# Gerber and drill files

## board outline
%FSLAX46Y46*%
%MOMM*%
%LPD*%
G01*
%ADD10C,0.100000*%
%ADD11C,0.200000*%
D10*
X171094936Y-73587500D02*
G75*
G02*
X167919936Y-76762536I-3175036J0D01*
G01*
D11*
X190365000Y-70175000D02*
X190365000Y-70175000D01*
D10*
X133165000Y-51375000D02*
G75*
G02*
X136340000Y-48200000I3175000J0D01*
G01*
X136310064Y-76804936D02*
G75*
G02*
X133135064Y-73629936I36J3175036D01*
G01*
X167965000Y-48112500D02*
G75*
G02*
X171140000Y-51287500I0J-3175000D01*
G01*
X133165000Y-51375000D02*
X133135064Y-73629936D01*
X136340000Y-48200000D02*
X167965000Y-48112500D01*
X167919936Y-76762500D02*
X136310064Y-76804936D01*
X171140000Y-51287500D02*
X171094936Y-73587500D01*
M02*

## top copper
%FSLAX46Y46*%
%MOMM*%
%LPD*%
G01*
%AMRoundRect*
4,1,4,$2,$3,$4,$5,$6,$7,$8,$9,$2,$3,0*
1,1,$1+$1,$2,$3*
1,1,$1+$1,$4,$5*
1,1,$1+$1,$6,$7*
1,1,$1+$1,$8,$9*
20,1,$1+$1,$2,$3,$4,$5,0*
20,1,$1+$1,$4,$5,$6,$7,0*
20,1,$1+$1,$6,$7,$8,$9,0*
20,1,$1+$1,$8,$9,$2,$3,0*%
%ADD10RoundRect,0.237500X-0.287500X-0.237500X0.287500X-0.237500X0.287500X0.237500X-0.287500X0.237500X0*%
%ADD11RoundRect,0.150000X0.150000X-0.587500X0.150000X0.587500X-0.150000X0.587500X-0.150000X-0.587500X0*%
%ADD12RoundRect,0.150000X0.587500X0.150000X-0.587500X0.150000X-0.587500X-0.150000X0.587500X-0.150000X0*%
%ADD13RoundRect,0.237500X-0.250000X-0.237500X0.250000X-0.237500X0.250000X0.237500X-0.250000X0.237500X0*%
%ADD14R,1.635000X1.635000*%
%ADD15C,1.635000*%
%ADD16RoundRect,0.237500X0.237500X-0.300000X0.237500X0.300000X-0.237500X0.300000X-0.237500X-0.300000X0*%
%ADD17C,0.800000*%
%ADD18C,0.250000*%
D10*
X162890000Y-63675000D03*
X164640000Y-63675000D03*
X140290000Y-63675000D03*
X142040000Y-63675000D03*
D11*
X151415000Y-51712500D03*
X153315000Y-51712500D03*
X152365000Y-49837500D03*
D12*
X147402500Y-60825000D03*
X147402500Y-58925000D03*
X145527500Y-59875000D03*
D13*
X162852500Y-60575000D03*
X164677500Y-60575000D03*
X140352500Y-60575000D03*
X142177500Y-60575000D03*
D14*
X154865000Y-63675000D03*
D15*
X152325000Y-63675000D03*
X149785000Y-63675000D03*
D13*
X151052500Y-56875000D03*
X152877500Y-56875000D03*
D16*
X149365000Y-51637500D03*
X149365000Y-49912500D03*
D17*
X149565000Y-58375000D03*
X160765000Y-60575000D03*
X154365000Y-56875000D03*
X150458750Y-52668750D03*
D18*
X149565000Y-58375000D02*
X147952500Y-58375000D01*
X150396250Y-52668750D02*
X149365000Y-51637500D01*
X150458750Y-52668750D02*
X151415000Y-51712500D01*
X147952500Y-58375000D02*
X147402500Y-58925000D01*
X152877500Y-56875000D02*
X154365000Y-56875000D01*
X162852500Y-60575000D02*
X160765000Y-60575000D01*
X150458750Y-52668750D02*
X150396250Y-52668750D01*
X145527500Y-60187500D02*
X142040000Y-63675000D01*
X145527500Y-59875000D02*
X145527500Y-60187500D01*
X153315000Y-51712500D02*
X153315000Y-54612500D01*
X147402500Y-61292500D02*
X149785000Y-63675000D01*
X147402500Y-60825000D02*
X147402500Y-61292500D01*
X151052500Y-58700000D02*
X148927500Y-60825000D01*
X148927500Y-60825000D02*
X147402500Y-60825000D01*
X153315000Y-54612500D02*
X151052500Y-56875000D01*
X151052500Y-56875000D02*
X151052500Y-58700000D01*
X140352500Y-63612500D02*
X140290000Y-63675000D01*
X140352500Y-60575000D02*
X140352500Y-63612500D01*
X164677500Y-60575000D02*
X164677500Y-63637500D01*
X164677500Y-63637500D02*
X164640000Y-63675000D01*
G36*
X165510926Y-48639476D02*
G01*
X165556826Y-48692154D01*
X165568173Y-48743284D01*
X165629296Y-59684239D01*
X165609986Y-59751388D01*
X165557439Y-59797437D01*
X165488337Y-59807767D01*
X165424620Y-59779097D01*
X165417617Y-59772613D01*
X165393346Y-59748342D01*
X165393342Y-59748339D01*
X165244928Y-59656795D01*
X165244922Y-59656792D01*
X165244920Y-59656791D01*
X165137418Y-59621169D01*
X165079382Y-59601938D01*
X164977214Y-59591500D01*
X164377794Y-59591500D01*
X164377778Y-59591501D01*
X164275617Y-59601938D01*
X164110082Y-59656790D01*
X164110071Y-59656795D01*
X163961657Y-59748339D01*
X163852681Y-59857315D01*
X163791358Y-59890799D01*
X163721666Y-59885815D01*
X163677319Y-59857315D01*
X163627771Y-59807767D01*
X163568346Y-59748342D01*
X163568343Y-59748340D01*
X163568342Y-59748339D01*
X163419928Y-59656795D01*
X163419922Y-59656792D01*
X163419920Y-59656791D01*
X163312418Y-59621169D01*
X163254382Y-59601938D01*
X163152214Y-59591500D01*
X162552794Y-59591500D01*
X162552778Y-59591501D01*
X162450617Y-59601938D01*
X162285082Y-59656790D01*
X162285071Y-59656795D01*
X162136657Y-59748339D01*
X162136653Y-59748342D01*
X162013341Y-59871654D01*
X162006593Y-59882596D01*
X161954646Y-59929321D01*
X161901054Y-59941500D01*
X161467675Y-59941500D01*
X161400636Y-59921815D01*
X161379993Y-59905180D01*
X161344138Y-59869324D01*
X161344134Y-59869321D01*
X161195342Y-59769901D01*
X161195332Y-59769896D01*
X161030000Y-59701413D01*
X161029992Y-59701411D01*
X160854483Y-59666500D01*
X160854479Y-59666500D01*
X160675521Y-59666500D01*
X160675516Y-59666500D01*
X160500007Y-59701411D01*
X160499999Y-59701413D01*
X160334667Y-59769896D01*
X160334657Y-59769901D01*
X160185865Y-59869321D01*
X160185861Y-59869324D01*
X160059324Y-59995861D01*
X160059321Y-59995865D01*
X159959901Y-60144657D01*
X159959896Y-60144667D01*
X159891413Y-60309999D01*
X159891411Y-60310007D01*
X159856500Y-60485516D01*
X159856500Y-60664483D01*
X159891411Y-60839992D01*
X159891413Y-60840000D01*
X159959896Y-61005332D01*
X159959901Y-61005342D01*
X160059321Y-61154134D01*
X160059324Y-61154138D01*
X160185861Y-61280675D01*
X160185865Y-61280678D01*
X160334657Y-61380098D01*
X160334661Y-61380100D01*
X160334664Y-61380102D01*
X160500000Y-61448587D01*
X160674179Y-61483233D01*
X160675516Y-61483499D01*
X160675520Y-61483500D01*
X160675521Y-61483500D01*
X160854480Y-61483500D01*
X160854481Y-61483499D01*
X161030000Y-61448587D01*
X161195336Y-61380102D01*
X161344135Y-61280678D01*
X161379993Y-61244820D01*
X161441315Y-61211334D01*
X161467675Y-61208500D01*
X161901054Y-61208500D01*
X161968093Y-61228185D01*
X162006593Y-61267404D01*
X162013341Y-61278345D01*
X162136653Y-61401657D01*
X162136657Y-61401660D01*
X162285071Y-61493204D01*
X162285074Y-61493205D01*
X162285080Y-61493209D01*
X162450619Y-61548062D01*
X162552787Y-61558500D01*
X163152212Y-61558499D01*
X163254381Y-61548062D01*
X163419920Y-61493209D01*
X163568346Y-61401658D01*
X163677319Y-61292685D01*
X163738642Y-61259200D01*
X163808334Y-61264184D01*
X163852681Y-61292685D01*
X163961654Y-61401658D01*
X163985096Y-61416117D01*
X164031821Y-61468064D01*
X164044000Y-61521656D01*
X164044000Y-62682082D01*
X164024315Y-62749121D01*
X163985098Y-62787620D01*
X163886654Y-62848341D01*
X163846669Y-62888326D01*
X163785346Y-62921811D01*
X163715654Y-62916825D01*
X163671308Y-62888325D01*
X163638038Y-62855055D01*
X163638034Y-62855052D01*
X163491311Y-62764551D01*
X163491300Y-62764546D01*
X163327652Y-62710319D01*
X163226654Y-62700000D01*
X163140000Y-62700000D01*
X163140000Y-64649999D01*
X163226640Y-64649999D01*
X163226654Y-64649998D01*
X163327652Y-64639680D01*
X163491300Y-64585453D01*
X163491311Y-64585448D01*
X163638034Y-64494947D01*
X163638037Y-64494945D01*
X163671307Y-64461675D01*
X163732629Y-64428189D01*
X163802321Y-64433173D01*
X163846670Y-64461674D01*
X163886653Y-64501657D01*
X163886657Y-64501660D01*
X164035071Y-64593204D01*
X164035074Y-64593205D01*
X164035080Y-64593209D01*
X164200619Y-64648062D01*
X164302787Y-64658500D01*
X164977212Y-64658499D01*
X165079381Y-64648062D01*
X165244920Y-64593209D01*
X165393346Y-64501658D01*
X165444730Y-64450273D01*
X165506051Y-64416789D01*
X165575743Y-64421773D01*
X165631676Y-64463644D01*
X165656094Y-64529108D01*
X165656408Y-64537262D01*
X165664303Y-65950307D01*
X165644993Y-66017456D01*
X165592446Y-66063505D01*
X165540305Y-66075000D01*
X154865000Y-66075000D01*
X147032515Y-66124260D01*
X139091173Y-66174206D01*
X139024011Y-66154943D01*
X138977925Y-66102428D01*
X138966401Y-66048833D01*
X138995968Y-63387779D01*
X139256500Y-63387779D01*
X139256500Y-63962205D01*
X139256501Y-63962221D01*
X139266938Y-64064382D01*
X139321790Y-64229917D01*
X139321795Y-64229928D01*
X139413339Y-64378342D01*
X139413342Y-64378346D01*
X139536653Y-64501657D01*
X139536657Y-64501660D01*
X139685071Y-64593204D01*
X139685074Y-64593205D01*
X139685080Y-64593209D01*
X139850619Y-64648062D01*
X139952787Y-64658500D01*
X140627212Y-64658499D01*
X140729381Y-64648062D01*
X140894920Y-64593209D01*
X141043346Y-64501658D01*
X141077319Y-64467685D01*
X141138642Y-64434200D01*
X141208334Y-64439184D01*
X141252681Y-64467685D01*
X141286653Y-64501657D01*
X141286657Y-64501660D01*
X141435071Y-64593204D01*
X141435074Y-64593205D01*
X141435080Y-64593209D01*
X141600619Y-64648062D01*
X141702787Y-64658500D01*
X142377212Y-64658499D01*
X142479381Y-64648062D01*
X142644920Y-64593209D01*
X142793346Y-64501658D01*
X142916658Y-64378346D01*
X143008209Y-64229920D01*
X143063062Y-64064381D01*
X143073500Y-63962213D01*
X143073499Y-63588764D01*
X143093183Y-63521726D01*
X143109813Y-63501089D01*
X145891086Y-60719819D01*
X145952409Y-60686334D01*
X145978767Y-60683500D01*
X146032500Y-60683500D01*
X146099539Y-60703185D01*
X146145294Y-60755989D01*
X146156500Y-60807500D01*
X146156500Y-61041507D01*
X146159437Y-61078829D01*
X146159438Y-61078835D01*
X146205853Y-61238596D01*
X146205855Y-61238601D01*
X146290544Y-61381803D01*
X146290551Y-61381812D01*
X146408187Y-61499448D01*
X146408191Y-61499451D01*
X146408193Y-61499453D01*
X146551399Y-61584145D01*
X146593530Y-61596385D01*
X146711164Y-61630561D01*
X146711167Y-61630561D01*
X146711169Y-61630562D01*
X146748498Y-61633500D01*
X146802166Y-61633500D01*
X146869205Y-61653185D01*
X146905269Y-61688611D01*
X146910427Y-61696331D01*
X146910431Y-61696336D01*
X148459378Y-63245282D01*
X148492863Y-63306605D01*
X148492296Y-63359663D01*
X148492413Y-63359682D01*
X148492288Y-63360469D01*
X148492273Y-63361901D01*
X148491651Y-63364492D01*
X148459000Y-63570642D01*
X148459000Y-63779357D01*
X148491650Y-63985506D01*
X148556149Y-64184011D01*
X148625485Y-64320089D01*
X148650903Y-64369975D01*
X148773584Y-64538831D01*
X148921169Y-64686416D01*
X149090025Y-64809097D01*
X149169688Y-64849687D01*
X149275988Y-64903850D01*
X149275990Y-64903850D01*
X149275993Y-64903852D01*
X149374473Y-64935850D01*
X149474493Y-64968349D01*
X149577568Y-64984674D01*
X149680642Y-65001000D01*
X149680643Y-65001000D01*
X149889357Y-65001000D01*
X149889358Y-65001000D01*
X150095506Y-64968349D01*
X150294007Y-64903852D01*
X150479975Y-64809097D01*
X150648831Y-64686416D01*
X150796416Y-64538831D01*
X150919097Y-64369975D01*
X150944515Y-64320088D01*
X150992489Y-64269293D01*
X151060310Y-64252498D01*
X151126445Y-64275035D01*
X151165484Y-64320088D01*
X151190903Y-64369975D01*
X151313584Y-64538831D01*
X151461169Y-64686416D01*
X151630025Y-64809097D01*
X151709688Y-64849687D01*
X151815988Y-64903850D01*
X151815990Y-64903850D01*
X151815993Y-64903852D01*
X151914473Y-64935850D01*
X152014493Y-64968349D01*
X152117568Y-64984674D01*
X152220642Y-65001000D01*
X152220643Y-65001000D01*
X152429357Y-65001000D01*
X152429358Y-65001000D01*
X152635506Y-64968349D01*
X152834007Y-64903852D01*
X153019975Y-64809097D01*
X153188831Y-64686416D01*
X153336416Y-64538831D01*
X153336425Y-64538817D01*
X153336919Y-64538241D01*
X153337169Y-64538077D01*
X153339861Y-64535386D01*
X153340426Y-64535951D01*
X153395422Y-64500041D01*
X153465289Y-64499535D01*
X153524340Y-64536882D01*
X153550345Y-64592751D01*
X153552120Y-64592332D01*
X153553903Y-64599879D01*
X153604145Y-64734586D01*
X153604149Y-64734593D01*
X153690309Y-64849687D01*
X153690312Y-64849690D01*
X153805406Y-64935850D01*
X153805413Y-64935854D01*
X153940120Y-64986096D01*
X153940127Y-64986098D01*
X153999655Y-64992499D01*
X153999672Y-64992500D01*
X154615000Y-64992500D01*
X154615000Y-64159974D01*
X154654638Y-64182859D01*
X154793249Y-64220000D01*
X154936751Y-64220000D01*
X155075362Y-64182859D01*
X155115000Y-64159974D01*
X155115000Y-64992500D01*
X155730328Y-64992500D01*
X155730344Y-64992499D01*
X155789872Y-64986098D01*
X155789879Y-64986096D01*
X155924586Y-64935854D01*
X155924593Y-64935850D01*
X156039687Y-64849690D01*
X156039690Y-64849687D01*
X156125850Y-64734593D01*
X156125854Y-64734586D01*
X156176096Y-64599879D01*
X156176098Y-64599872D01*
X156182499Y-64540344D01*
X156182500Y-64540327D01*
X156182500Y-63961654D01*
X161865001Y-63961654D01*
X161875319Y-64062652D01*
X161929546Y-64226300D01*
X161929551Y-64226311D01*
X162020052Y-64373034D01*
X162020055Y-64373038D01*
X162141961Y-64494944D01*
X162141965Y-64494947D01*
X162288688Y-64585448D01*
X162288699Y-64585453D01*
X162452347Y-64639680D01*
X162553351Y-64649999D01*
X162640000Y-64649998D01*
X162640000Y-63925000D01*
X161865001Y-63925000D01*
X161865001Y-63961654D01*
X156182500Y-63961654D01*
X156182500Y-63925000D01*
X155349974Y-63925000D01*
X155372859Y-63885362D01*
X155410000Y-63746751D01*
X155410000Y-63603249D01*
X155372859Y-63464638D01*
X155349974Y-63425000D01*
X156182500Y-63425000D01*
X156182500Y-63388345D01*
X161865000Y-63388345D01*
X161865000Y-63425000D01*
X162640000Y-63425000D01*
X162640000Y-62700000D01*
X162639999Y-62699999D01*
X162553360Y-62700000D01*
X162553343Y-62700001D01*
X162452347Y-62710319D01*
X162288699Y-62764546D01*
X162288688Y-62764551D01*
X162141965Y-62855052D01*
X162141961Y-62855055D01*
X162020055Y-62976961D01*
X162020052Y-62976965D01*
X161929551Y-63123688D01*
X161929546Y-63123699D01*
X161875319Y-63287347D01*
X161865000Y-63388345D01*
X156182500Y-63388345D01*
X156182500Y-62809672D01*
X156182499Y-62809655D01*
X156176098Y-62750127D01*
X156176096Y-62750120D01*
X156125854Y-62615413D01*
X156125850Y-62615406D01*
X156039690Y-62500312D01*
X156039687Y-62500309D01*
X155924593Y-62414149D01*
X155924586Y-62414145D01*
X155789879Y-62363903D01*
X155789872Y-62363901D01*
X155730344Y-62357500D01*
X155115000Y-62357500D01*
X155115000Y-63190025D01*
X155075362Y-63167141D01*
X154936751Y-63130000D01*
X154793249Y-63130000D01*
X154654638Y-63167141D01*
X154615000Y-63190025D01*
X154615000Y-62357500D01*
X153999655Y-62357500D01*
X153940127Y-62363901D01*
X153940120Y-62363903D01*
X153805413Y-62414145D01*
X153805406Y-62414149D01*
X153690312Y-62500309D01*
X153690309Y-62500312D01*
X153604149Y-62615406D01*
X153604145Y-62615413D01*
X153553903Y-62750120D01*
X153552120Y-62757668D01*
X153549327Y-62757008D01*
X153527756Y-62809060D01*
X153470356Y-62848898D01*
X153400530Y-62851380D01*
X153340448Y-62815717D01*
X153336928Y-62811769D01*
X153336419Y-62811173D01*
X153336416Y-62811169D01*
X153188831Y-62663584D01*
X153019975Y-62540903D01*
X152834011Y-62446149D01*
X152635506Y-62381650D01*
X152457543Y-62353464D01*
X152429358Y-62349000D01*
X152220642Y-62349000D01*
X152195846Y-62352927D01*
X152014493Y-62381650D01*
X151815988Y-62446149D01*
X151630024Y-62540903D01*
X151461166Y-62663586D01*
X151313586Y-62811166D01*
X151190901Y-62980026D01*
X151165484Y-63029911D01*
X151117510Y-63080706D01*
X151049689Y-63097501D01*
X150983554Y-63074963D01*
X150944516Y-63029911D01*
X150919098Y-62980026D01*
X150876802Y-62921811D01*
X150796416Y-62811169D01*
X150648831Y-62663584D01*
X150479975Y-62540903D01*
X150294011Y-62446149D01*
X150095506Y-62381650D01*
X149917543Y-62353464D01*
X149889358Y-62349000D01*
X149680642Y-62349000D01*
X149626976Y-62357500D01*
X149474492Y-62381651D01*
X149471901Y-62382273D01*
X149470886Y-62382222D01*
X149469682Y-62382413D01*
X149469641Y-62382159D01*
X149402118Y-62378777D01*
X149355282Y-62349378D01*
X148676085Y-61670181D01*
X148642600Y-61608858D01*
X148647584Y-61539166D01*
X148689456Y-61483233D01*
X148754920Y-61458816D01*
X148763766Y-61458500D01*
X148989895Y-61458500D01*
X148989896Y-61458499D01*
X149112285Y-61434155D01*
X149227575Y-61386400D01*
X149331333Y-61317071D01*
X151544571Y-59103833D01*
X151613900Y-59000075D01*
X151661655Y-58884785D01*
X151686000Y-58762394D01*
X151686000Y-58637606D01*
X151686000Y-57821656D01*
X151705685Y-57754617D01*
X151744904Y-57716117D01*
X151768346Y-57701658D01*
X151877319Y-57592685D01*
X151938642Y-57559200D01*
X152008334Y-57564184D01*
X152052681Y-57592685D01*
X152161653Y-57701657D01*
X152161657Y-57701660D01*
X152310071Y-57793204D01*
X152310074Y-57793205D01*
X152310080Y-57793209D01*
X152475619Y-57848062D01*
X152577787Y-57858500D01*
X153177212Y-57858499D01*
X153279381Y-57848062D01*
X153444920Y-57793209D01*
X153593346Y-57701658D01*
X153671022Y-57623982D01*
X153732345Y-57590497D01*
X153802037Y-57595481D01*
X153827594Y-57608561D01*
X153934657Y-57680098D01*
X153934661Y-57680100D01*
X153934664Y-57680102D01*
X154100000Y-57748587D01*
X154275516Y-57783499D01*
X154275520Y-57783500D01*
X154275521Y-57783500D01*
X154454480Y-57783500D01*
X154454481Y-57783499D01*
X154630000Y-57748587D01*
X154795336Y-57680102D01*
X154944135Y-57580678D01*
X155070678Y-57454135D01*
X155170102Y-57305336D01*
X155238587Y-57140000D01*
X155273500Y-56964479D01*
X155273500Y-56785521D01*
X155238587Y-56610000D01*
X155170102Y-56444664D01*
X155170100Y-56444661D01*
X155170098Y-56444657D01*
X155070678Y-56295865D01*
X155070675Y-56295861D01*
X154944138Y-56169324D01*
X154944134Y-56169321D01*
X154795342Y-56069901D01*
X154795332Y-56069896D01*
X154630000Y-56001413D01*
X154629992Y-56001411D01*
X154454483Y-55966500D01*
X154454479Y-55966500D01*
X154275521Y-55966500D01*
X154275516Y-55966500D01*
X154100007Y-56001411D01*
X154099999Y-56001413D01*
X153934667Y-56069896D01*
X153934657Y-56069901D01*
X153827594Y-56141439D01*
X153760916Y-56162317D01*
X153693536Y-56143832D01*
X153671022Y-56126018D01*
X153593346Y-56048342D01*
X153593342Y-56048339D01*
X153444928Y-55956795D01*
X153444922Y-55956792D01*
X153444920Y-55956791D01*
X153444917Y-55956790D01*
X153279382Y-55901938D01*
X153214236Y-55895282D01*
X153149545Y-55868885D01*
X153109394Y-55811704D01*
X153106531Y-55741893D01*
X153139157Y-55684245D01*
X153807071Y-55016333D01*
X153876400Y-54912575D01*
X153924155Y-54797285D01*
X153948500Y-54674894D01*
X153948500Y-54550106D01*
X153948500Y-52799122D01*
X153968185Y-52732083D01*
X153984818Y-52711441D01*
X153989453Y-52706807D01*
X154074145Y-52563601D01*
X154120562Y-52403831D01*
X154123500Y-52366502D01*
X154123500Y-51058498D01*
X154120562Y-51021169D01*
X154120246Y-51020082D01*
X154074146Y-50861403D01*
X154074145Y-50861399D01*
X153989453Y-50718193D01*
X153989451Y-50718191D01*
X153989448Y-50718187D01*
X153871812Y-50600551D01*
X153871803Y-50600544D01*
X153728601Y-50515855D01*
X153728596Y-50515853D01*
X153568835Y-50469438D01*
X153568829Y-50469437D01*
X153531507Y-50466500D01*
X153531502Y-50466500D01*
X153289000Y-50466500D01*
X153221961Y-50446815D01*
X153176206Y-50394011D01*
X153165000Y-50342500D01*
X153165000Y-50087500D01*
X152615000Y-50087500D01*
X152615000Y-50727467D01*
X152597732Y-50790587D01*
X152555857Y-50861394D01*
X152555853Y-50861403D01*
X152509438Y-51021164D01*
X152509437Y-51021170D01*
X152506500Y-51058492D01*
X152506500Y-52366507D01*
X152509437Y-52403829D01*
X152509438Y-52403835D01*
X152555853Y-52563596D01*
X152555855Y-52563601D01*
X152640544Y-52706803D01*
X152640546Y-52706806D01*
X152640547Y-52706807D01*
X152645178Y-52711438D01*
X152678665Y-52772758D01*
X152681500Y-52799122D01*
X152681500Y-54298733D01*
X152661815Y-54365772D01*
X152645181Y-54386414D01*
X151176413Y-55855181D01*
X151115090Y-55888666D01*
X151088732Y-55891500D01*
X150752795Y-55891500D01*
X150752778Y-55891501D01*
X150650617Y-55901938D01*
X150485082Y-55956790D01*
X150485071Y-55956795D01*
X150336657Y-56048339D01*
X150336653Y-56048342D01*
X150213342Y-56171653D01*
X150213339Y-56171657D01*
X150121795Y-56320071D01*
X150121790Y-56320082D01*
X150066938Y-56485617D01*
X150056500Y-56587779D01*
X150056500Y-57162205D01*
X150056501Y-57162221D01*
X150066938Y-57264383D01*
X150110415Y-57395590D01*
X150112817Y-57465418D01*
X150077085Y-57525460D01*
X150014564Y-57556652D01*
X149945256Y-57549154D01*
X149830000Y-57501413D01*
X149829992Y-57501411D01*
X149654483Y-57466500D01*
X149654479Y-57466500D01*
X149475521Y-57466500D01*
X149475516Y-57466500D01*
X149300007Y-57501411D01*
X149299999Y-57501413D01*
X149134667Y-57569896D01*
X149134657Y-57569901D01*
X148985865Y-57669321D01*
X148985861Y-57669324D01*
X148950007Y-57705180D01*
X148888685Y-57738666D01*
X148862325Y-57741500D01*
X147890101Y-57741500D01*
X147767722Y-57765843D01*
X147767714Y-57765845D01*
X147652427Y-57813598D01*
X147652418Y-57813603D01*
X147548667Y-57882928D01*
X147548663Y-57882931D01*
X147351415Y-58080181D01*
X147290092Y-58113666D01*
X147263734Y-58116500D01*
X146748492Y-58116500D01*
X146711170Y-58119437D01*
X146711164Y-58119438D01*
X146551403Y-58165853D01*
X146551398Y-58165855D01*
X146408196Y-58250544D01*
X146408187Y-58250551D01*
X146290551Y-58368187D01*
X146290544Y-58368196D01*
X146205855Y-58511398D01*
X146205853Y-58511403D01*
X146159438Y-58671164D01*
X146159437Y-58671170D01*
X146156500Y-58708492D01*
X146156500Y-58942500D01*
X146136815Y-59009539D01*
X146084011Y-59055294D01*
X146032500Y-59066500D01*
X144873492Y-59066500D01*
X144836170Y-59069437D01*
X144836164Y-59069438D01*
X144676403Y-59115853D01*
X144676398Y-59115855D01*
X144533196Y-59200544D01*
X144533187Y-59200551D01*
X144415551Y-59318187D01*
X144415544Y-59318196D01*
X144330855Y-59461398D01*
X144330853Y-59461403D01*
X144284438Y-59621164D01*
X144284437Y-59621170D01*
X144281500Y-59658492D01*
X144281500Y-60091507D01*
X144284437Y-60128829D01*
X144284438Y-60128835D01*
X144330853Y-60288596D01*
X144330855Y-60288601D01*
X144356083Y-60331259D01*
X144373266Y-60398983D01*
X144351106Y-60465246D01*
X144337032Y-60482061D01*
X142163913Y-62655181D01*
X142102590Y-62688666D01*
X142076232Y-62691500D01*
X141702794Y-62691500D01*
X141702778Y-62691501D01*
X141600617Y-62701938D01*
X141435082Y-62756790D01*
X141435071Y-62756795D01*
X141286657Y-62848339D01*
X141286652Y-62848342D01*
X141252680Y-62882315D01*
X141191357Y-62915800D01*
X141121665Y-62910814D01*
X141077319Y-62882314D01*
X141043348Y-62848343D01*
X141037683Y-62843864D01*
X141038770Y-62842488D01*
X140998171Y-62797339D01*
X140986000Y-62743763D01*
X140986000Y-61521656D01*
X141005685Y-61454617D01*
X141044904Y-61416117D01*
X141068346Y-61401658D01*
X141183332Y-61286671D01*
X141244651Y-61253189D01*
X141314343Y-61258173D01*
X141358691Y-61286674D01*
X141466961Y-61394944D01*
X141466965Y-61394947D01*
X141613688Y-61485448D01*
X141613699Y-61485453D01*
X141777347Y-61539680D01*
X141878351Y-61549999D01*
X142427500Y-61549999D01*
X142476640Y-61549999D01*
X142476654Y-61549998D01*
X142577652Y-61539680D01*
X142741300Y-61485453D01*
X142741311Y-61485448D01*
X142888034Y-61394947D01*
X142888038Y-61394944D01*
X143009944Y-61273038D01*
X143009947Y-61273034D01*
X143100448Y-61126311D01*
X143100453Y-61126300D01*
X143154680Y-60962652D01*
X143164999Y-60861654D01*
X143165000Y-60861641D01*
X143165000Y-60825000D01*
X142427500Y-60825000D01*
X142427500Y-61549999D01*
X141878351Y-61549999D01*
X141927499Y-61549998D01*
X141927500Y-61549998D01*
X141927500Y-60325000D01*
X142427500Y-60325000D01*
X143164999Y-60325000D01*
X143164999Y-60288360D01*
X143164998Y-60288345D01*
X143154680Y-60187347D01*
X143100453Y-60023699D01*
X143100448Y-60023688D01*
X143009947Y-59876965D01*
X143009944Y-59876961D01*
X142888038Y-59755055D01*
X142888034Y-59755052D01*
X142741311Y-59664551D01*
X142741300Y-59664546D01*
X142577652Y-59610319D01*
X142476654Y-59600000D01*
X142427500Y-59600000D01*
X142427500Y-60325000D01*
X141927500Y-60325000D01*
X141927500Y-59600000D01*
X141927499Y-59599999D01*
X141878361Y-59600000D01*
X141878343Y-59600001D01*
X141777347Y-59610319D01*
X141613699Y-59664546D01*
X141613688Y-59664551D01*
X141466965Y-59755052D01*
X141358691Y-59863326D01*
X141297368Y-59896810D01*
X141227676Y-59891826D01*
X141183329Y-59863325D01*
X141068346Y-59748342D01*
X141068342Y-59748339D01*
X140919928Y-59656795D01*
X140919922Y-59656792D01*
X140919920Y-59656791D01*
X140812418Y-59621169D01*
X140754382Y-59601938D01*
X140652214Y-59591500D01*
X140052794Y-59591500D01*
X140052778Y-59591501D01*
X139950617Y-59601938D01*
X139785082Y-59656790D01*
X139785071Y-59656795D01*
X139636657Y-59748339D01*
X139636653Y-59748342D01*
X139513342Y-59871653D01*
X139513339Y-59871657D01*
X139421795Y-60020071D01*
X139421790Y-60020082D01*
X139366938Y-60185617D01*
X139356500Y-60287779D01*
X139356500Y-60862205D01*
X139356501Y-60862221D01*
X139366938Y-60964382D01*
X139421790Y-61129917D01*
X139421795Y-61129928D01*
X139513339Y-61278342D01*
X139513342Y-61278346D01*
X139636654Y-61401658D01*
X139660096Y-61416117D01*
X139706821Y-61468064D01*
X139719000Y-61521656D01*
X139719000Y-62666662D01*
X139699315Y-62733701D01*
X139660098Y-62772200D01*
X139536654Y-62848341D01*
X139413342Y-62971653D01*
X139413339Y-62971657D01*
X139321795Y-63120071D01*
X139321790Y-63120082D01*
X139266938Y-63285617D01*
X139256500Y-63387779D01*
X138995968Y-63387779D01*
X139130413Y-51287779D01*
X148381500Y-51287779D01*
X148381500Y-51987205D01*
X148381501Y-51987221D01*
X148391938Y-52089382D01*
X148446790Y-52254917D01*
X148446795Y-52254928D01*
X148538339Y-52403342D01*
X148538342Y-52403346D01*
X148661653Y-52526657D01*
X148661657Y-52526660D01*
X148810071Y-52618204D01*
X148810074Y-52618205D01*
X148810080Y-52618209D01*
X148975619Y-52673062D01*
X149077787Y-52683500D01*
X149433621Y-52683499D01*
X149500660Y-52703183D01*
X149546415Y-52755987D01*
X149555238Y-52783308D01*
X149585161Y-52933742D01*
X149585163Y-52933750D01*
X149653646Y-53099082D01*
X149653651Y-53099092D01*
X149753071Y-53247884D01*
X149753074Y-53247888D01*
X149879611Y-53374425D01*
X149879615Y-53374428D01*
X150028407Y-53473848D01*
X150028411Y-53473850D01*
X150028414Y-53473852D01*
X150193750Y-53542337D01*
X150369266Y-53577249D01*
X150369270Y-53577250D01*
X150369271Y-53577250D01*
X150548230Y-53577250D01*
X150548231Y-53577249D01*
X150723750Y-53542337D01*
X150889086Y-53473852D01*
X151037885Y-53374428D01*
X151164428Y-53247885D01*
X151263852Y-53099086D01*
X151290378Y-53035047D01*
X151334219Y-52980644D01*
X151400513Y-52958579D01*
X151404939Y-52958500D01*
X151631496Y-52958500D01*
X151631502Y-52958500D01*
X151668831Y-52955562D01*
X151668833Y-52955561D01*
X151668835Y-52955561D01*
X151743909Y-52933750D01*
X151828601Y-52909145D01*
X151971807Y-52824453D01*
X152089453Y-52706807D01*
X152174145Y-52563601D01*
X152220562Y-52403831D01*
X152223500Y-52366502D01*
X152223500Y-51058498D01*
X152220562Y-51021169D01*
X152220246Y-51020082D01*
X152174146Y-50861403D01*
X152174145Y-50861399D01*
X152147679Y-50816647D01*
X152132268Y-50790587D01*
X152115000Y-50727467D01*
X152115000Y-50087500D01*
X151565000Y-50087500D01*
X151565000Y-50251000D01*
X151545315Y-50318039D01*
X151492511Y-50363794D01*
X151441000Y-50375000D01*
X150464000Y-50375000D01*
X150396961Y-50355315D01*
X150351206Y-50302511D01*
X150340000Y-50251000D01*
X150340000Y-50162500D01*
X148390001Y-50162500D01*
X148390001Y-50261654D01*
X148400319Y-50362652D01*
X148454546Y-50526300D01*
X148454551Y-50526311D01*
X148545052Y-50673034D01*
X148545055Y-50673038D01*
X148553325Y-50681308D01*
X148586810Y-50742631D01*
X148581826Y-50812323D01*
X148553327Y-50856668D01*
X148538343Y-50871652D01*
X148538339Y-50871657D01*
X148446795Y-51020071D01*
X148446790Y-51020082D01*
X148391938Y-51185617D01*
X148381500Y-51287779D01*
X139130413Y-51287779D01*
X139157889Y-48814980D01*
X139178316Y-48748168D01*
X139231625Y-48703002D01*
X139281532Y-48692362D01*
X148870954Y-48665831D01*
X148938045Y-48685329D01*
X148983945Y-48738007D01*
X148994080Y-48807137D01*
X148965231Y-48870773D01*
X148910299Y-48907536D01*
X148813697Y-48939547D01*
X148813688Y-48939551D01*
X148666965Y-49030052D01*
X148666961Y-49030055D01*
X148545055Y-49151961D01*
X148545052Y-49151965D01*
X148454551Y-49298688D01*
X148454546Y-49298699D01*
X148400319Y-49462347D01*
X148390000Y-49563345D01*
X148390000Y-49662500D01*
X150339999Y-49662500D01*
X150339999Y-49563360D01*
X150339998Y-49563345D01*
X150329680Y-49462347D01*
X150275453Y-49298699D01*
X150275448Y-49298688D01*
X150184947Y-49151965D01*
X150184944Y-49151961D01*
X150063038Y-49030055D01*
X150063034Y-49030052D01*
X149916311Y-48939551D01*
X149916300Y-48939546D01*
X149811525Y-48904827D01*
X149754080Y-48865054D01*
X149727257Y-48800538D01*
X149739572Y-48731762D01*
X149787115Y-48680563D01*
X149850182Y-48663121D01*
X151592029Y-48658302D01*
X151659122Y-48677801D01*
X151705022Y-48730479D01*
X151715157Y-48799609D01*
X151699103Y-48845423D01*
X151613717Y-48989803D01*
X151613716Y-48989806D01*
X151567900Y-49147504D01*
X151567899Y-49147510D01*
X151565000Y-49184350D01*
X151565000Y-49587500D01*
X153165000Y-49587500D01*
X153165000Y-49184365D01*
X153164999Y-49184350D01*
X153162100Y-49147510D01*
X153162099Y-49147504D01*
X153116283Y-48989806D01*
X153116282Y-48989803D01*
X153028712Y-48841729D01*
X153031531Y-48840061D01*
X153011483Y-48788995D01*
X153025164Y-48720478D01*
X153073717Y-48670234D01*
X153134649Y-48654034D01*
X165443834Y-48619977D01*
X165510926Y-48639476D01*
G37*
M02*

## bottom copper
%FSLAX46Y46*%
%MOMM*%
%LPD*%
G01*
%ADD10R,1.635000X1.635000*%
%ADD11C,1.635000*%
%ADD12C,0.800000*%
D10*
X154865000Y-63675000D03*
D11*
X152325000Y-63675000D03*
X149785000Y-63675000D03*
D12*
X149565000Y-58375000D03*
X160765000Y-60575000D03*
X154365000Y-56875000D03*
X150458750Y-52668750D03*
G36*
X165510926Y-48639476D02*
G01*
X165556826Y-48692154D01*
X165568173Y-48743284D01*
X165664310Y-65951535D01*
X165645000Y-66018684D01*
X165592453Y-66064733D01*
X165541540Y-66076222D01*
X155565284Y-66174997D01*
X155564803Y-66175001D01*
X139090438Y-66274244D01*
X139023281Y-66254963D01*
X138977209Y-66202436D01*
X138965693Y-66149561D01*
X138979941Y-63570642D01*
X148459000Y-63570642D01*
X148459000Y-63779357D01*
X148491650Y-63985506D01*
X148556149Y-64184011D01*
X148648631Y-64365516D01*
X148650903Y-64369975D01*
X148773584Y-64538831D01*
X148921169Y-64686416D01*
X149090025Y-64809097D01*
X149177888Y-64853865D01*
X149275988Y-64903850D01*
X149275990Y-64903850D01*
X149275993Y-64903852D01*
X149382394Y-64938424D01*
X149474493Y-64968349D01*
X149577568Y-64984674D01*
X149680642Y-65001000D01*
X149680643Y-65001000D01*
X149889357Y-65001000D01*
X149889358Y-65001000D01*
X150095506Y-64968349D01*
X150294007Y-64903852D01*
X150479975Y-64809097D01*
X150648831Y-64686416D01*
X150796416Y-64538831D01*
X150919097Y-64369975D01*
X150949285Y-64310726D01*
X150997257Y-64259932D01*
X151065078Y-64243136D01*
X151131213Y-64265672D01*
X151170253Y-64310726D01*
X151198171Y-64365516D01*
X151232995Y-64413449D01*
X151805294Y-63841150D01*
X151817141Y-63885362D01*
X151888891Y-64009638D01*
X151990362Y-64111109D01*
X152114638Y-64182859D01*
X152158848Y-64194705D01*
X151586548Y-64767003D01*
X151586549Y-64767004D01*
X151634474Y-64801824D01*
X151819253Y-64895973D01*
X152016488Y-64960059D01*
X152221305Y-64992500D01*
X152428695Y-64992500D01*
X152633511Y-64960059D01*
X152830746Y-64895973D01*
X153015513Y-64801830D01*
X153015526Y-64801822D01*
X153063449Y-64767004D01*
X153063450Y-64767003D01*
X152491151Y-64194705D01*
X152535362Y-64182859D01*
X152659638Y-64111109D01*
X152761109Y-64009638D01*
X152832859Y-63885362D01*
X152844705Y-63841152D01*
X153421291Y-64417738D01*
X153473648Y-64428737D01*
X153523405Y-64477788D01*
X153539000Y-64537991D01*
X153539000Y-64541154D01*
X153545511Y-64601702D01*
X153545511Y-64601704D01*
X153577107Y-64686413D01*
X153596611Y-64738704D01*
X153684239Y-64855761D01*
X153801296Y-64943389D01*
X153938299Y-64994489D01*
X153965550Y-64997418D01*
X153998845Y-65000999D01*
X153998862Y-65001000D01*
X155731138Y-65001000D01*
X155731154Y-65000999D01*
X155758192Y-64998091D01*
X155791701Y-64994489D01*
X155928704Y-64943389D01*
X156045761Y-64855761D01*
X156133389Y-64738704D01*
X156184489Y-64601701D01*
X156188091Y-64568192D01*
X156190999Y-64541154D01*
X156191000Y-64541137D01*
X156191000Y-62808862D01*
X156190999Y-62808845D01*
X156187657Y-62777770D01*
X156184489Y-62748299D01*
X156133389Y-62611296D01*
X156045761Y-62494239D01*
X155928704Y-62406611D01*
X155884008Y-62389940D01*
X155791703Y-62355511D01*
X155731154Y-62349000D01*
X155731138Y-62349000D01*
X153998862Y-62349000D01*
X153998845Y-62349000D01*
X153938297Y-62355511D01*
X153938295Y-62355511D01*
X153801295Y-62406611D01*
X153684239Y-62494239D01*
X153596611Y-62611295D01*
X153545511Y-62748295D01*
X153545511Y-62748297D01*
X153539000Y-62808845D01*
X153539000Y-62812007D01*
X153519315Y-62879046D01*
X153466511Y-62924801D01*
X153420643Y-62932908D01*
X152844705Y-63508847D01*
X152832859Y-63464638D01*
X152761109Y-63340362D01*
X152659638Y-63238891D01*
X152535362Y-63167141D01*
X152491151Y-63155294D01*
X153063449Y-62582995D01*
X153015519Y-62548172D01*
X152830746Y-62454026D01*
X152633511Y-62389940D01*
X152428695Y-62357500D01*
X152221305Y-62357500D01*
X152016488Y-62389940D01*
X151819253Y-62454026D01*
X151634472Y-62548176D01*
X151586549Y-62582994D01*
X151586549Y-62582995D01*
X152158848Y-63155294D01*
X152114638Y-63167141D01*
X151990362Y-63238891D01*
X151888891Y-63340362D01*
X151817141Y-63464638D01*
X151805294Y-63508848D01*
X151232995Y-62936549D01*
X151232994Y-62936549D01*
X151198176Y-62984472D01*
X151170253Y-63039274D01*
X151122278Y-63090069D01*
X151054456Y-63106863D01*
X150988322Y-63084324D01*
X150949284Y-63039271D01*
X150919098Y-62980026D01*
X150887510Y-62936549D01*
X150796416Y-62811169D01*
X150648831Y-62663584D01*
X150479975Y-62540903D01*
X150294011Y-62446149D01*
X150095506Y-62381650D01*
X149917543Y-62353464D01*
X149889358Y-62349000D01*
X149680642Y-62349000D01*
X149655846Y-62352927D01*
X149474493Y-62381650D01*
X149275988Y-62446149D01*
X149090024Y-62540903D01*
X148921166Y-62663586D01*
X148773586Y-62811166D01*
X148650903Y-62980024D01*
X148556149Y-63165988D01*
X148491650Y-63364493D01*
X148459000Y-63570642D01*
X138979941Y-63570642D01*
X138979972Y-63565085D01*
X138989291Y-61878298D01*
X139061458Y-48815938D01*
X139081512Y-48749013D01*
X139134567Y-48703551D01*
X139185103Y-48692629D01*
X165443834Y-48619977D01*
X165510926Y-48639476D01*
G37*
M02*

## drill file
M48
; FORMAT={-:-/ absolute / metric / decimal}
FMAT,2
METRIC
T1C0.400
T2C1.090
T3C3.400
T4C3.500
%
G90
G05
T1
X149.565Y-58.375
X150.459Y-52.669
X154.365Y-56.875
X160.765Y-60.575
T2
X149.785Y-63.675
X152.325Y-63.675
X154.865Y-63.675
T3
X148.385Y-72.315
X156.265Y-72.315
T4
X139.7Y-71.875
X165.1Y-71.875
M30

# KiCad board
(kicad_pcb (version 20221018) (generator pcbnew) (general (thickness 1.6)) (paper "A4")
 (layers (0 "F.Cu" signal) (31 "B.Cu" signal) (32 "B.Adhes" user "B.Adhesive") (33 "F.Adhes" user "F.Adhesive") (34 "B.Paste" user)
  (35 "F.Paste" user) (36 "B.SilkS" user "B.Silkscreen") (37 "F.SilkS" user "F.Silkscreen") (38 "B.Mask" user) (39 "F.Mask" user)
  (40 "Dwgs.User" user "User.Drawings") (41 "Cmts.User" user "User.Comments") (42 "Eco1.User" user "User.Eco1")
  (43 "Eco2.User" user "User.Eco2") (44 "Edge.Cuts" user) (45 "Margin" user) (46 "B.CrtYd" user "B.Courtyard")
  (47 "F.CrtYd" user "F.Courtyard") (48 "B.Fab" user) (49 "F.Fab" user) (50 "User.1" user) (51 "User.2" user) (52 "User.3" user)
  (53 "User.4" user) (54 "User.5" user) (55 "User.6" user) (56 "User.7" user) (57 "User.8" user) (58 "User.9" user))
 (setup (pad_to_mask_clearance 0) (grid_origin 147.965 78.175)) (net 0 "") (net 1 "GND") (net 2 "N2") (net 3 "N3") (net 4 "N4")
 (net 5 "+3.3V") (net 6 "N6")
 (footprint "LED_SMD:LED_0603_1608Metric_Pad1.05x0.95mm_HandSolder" (layer "F.Cu") (at 163.765 63.675)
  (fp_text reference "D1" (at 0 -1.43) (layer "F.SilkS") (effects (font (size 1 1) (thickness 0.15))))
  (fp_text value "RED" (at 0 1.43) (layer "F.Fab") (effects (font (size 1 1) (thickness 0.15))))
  (pad "1" smd roundrect (at -0.875 0) (size 1.05 0.95) (layers "F.Cu" "F.Paste" "F.Mask") (roundrect_rratio 0.25) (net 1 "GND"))
  (pad "2" smd roundrect (at 0.875 0) (size 1.05 0.95) (layers "F.Cu" "F.Paste" "F.Mask") (roundrect_rratio 0.25) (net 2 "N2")))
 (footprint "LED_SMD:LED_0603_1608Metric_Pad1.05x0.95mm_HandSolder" (layer "F.Cu") (at 141.165 63.675)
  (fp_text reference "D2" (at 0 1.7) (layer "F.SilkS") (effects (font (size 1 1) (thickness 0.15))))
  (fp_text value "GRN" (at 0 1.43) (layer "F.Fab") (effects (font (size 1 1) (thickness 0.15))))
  (pad "1" smd roundrect (at -0.875 0) (size 1.05 0.95) (layers "F.Cu" "F.Paste" "F.Mask") (roundrect_rratio 0.25) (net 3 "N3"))
  (pad "2" smd roundrect (at 0.875 0) (size 1.05 0.95) (layers "F.Cu" "F.Paste" "F.Mask") (roundrect_rratio 0.25) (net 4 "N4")))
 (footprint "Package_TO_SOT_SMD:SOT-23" (layer "F.Cu") (at 152.365 50.775 90)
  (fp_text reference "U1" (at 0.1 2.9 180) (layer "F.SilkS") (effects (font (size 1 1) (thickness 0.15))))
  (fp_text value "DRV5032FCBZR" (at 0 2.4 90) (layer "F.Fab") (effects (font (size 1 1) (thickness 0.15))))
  (pad "1" smd roundrect (at -0.9375 -0.95 90) (size 1.475 0.6) (layers "F.Cu" "F.Paste" "F.Mask") (roundrect_rratio 0.25) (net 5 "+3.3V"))
  (pad "2" smd roundrect (at -0.9375 0.95 90) (size 1.475 0.6) (layers "F.Cu" "F.Paste" "F.Mask") (roundrect_rratio 0.25) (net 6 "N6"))
  (pad "3" smd roundrect (at 0.9375 0 90) (size 1.475 0.6) (layers "F.Cu" "F.Paste" "F.Mask") (roundrect_rratio 0.25) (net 1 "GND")))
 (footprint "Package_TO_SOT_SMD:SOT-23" (layer "F.Cu") (at 146.465 59.875 180)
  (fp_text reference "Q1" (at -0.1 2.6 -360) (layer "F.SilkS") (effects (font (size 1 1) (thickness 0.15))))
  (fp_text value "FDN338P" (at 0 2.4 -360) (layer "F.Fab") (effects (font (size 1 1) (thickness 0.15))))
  (pad "1" smd roundrect (at -0.9375 -0.95 180) (size 1.475 0.6) (layers "F.Cu" "F.Paste" "F.Mask") (roundrect_rratio 0.25) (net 6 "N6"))
  (pad "2" smd roundrect (at -0.9375 0.95 180) (size 1.475 0.6) (layers "F.Cu" "F.Paste" "F.Mask") (roundrect_rratio 0.25) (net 5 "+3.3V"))
  (pad "3" smd roundrect (at 0.9375 0 180) (size 1.475 0.6) (layers "F.Cu" "F.Paste" "F.Mask") (roundrect_rratio 0.25) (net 4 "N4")))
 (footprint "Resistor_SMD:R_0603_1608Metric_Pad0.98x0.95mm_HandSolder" (layer "F.Cu") (at 163.765 60.575)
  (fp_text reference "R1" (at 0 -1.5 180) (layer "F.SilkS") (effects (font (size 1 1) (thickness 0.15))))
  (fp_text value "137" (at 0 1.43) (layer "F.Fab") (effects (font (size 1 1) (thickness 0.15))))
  (pad "1" smd roundrect (at -0.9125 0) (size 0.975 0.95) (layers "F.Cu" "F.Paste" "F.Mask") (roundrect_rratio 0.25) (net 5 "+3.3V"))
  (pad "2" smd roundrect (at 0.9125 0) (size 0.975 0.95) (layers "F.Cu" "F.Paste" "F.Mask") (roundrect_rratio 0.25) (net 2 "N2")))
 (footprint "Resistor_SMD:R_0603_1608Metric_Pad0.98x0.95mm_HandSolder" (layer "F.Cu") (at 141.265 60.575)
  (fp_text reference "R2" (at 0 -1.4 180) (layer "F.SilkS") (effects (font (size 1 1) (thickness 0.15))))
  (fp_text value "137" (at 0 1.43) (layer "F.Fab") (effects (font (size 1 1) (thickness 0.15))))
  (pad "1" smd roundrect (at -0.9125 0) (size 0.975 0.95) (layers "F.Cu" "F.Paste" "F.Mask") (roundrect_rratio 0.25) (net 3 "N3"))
  (pad "2" smd roundrect (at 0.9125 0) (size 0.975 0.95) (layers "F.Cu" "F.Paste" "F.Mask") (roundrect_rratio 0.25) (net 1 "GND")))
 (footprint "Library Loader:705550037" (layer "F.Cu") (at 154.865 63.675)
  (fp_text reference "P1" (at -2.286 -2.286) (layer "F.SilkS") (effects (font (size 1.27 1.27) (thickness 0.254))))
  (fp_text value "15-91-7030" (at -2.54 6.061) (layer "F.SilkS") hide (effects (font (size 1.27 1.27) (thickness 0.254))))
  (pad "" np_thru_hole circle (at -6.48 8.64) (size 0.001 0.001) (drill 3.4) (layers "*.Cu" "*.Mask"))
  (pad "" np_thru_hole circle (at 1.4 8.64) (size 0.001 0.001) (drill 3.4) (layers "*.Cu" "*.Mask"))
  (pad "1" thru_hole rect (at 0 0) (size 1.635 1.635) (drill 1.09) (layers "*.Cu" "*.Mask") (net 1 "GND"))
  (pad "2" thru_hole circle (at -2.54 0) (size 1.635 1.635) (drill 1.09) (layers "*.Cu" "*.Mask") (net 5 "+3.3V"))
  (pad "3" thru_hole circle (at -5.08 0) (size 1.635 1.635) (drill 1.09) (layers "*.Cu" "*.Mask") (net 6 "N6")))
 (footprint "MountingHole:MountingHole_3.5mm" (layer "F.Cu") (at 165.1 71.875)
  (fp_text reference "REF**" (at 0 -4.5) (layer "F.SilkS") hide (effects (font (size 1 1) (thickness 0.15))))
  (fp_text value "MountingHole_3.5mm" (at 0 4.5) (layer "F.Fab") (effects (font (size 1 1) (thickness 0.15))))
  (pad "" np_thru_hole circle (at 0 0) (size 3.5 3.5) (drill 3.5) (layers "*.Cu" "*.Mask")))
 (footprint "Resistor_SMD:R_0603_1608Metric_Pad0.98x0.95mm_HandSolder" (layer "F.Cu") (at 151.965 56.875)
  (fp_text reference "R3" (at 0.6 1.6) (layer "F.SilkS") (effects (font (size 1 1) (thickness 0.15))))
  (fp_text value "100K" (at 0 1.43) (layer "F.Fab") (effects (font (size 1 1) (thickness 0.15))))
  (pad "1" smd roundrect (at -0.9125 0) (size 0.975 0.95) (layers "F.Cu" "F.Paste" "F.Mask") (roundrect_rratio 0.25) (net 6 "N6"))
  (pad "2" smd roundrect (at 0.9125 0) (size 0.975 0.95) (layers "F.Cu" "F.Paste" "F.Mask") (roundrect_rratio 0.25) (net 5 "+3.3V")))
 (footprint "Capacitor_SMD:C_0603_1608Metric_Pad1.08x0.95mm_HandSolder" (layer "F.Cu") (at 149.365 50.775 90)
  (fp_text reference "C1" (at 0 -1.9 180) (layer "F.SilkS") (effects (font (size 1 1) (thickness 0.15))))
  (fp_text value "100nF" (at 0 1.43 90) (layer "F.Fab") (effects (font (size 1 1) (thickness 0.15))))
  (pad "1" smd roundrect (at -0.8625 0 90) (size 1.075 0.95) (layers "F.Cu" "F.Paste" "F.Mask") (roundrect_rratio 0.25) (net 5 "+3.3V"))
  (pad "2" smd roundrect (at 0.8625 0 90) (size 1.075 0.95) (layers "F.Cu" "F.Paste" "F.Mask") (roundrect_rratio 0.25) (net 1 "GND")))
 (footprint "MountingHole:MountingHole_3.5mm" (layer "F.Cu") (at 139.7 71.875)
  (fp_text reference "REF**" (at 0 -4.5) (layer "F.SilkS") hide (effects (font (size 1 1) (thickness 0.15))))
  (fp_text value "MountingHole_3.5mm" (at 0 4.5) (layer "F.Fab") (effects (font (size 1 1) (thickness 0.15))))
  (pad "" np_thru_hole circle (at 0 0) (size 3.5 3.5) (drill 3.5) (layers "*.Cu" "*.Mask")))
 (gr_arc (start 171.094936 73.5875) (mid 170.165 75.832564) (end 167.919936 76.7625) (stroke (width 0.1) (type default)) (layer "Edge.Cuts"))
 (gr_line (start 190.365 70.175) (end 190.365 70.175) (stroke (width 0.2) (type default)) (layer "Edge.Cuts"))
 (gr_arc (start 133.165 51.375) (mid 134.094936 49.129936) (end 136.34 48.2) (stroke (width 0.1) (type default)) (layer "Edge.Cuts"))
 (gr_arc (start 136.310064 76.804936) (mid 134.065 75.875) (end 133.135064 73.629936) (stroke (width 0.1) (type default))
  (layer "Edge.Cuts"))
 (gr_arc (start 167.965 48.1125) (mid 170.210064 49.042436) (end 171.14 51.2875) (stroke (width 0.1) (type default)) (layer "Edge.Cuts"))
 (gr_line (start 133.165 51.375) (end 133.135064 73.629936) (stroke (width 0.1) (type default)) (layer "Edge.Cuts"))
 (gr_line (start 136.34 48.2) (end 167.965 48.1125) (stroke (width 0.1) (type default)) (layer "Edge.Cuts"))
 (gr_line (start 167.919936 76.7625) (end 136.310064 76.804936) (stroke (width 0.1) (type default)) (layer "Edge.Cuts"))
 (gr_line (start 171.14 51.2875) (end 171.094936 73.5875) (stroke (width 0.1) (type default)) (layer "Edge.Cuts"))
 (segment (start 149.565 58.375) (end 147.9525 58.375) (width 0.25) (layer "F.Cu") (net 5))
 (segment (start 150.39625 52.66875) (end 149.365 51.6375) (width 0.25) (layer "F.Cu") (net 5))
 (segment (start 150.45875 52.66875) (end 151.415 51.7125) (width 0.25) (layer "F.Cu") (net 5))
 (segment (start 147.9525 58.375) (end 147.4025 58.925) (width 0.25) (layer "F.Cu") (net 5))
 (segment (start 152.8775 56.875) (end 154.365 56.875) (width 0.25) (layer "F.Cu") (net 5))
 (segment (start 162.8525 60.575) (end 160.765 60.575) (width 0.25) (layer "F.Cu") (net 5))
 (segment (start 150.45875 52.66875) (end 150.39625 52.66875) (width 0.25) (layer "F.Cu") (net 5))
 (via (at 149.565 58.375) (size 0.8) (drill 0.4) (layers "F.Cu" "B.Cu") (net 5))
 (via (at 160.765 60.575) (size 0.8) (drill 0.4) (layers "F.Cu" "B.Cu") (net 5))
 (via (at 154.365 56.875) (size 0.8) (drill 0.4) (layers "F.Cu" "B.Cu") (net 5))
 (via (at 150.45875 52.66875) (size 0.8) (drill 0.4) (layers "F.Cu" "B.Cu") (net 5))
 (segment (start 145.5275 60.1875) (end 142.04 63.675) (width 0.25) (layer "F.Cu") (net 4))
 (segment (start 145.5275 59.875) (end 145.5275 60.1875) (width 0.25) (layer "F.Cu") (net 4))
 (segment (start 153.315 51.7125) (end 153.315 54.6125) (width 0.25) (layer "F.Cu") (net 6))
 (segment (start 147.4025 61.2925) (end 149.785 63.675) (width 0.25) (layer "F.Cu") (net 6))
 (segment (start 147.4025 60.825) (end 147.4025 61.2925) (width 0.25) (layer "F.Cu") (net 6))
 (segment (start 151.0525 58.7) (end 148.9275 60.825) (width 0.25) (layer "F.Cu") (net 6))
 (segment (start 148.9275 60.825) (end 147.4025 60.825) (width 0.25) (layer "F.Cu") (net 6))
 (segment (start 153.315 54.6125) (end 151.0525 56.875) (width 0.25) (layer "F.Cu") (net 6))
 (segment (start 151.0525 56.875) (end 151.0525 58.7) (width 0.25) (layer "F.Cu") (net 6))
 (segment (start 140.3525 63.6125) (end 140.29 63.675) (width 0.25) (layer "F.Cu") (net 3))
 (segment (start 140.3525 60.575) (end 140.3525 63.6125) (width 0.25) (layer "F.Cu") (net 3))
 (segment (start 164.6775 60.575) (end 164.6775 63.6375) (width 0.25) (layer "F.Cu") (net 2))
 (segment (start 164.6775 63.6375) (end 164.64 63.675) (width 0.25) (layer "F.Cu") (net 2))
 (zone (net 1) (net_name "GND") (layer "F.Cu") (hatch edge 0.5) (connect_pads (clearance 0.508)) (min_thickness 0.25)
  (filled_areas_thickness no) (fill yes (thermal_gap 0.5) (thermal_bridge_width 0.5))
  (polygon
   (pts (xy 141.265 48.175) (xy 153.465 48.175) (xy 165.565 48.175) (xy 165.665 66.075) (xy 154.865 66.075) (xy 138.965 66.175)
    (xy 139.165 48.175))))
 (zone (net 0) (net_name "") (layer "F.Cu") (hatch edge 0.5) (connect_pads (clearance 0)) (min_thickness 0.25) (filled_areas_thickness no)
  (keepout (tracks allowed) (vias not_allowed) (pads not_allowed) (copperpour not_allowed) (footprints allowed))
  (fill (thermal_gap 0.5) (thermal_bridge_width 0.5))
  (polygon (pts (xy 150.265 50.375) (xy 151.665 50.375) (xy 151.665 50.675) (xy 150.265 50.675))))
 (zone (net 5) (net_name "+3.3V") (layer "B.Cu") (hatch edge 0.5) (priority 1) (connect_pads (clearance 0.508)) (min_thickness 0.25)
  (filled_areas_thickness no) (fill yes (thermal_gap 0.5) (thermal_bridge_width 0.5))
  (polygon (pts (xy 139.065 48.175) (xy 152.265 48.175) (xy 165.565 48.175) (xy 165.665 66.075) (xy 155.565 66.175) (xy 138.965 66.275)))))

